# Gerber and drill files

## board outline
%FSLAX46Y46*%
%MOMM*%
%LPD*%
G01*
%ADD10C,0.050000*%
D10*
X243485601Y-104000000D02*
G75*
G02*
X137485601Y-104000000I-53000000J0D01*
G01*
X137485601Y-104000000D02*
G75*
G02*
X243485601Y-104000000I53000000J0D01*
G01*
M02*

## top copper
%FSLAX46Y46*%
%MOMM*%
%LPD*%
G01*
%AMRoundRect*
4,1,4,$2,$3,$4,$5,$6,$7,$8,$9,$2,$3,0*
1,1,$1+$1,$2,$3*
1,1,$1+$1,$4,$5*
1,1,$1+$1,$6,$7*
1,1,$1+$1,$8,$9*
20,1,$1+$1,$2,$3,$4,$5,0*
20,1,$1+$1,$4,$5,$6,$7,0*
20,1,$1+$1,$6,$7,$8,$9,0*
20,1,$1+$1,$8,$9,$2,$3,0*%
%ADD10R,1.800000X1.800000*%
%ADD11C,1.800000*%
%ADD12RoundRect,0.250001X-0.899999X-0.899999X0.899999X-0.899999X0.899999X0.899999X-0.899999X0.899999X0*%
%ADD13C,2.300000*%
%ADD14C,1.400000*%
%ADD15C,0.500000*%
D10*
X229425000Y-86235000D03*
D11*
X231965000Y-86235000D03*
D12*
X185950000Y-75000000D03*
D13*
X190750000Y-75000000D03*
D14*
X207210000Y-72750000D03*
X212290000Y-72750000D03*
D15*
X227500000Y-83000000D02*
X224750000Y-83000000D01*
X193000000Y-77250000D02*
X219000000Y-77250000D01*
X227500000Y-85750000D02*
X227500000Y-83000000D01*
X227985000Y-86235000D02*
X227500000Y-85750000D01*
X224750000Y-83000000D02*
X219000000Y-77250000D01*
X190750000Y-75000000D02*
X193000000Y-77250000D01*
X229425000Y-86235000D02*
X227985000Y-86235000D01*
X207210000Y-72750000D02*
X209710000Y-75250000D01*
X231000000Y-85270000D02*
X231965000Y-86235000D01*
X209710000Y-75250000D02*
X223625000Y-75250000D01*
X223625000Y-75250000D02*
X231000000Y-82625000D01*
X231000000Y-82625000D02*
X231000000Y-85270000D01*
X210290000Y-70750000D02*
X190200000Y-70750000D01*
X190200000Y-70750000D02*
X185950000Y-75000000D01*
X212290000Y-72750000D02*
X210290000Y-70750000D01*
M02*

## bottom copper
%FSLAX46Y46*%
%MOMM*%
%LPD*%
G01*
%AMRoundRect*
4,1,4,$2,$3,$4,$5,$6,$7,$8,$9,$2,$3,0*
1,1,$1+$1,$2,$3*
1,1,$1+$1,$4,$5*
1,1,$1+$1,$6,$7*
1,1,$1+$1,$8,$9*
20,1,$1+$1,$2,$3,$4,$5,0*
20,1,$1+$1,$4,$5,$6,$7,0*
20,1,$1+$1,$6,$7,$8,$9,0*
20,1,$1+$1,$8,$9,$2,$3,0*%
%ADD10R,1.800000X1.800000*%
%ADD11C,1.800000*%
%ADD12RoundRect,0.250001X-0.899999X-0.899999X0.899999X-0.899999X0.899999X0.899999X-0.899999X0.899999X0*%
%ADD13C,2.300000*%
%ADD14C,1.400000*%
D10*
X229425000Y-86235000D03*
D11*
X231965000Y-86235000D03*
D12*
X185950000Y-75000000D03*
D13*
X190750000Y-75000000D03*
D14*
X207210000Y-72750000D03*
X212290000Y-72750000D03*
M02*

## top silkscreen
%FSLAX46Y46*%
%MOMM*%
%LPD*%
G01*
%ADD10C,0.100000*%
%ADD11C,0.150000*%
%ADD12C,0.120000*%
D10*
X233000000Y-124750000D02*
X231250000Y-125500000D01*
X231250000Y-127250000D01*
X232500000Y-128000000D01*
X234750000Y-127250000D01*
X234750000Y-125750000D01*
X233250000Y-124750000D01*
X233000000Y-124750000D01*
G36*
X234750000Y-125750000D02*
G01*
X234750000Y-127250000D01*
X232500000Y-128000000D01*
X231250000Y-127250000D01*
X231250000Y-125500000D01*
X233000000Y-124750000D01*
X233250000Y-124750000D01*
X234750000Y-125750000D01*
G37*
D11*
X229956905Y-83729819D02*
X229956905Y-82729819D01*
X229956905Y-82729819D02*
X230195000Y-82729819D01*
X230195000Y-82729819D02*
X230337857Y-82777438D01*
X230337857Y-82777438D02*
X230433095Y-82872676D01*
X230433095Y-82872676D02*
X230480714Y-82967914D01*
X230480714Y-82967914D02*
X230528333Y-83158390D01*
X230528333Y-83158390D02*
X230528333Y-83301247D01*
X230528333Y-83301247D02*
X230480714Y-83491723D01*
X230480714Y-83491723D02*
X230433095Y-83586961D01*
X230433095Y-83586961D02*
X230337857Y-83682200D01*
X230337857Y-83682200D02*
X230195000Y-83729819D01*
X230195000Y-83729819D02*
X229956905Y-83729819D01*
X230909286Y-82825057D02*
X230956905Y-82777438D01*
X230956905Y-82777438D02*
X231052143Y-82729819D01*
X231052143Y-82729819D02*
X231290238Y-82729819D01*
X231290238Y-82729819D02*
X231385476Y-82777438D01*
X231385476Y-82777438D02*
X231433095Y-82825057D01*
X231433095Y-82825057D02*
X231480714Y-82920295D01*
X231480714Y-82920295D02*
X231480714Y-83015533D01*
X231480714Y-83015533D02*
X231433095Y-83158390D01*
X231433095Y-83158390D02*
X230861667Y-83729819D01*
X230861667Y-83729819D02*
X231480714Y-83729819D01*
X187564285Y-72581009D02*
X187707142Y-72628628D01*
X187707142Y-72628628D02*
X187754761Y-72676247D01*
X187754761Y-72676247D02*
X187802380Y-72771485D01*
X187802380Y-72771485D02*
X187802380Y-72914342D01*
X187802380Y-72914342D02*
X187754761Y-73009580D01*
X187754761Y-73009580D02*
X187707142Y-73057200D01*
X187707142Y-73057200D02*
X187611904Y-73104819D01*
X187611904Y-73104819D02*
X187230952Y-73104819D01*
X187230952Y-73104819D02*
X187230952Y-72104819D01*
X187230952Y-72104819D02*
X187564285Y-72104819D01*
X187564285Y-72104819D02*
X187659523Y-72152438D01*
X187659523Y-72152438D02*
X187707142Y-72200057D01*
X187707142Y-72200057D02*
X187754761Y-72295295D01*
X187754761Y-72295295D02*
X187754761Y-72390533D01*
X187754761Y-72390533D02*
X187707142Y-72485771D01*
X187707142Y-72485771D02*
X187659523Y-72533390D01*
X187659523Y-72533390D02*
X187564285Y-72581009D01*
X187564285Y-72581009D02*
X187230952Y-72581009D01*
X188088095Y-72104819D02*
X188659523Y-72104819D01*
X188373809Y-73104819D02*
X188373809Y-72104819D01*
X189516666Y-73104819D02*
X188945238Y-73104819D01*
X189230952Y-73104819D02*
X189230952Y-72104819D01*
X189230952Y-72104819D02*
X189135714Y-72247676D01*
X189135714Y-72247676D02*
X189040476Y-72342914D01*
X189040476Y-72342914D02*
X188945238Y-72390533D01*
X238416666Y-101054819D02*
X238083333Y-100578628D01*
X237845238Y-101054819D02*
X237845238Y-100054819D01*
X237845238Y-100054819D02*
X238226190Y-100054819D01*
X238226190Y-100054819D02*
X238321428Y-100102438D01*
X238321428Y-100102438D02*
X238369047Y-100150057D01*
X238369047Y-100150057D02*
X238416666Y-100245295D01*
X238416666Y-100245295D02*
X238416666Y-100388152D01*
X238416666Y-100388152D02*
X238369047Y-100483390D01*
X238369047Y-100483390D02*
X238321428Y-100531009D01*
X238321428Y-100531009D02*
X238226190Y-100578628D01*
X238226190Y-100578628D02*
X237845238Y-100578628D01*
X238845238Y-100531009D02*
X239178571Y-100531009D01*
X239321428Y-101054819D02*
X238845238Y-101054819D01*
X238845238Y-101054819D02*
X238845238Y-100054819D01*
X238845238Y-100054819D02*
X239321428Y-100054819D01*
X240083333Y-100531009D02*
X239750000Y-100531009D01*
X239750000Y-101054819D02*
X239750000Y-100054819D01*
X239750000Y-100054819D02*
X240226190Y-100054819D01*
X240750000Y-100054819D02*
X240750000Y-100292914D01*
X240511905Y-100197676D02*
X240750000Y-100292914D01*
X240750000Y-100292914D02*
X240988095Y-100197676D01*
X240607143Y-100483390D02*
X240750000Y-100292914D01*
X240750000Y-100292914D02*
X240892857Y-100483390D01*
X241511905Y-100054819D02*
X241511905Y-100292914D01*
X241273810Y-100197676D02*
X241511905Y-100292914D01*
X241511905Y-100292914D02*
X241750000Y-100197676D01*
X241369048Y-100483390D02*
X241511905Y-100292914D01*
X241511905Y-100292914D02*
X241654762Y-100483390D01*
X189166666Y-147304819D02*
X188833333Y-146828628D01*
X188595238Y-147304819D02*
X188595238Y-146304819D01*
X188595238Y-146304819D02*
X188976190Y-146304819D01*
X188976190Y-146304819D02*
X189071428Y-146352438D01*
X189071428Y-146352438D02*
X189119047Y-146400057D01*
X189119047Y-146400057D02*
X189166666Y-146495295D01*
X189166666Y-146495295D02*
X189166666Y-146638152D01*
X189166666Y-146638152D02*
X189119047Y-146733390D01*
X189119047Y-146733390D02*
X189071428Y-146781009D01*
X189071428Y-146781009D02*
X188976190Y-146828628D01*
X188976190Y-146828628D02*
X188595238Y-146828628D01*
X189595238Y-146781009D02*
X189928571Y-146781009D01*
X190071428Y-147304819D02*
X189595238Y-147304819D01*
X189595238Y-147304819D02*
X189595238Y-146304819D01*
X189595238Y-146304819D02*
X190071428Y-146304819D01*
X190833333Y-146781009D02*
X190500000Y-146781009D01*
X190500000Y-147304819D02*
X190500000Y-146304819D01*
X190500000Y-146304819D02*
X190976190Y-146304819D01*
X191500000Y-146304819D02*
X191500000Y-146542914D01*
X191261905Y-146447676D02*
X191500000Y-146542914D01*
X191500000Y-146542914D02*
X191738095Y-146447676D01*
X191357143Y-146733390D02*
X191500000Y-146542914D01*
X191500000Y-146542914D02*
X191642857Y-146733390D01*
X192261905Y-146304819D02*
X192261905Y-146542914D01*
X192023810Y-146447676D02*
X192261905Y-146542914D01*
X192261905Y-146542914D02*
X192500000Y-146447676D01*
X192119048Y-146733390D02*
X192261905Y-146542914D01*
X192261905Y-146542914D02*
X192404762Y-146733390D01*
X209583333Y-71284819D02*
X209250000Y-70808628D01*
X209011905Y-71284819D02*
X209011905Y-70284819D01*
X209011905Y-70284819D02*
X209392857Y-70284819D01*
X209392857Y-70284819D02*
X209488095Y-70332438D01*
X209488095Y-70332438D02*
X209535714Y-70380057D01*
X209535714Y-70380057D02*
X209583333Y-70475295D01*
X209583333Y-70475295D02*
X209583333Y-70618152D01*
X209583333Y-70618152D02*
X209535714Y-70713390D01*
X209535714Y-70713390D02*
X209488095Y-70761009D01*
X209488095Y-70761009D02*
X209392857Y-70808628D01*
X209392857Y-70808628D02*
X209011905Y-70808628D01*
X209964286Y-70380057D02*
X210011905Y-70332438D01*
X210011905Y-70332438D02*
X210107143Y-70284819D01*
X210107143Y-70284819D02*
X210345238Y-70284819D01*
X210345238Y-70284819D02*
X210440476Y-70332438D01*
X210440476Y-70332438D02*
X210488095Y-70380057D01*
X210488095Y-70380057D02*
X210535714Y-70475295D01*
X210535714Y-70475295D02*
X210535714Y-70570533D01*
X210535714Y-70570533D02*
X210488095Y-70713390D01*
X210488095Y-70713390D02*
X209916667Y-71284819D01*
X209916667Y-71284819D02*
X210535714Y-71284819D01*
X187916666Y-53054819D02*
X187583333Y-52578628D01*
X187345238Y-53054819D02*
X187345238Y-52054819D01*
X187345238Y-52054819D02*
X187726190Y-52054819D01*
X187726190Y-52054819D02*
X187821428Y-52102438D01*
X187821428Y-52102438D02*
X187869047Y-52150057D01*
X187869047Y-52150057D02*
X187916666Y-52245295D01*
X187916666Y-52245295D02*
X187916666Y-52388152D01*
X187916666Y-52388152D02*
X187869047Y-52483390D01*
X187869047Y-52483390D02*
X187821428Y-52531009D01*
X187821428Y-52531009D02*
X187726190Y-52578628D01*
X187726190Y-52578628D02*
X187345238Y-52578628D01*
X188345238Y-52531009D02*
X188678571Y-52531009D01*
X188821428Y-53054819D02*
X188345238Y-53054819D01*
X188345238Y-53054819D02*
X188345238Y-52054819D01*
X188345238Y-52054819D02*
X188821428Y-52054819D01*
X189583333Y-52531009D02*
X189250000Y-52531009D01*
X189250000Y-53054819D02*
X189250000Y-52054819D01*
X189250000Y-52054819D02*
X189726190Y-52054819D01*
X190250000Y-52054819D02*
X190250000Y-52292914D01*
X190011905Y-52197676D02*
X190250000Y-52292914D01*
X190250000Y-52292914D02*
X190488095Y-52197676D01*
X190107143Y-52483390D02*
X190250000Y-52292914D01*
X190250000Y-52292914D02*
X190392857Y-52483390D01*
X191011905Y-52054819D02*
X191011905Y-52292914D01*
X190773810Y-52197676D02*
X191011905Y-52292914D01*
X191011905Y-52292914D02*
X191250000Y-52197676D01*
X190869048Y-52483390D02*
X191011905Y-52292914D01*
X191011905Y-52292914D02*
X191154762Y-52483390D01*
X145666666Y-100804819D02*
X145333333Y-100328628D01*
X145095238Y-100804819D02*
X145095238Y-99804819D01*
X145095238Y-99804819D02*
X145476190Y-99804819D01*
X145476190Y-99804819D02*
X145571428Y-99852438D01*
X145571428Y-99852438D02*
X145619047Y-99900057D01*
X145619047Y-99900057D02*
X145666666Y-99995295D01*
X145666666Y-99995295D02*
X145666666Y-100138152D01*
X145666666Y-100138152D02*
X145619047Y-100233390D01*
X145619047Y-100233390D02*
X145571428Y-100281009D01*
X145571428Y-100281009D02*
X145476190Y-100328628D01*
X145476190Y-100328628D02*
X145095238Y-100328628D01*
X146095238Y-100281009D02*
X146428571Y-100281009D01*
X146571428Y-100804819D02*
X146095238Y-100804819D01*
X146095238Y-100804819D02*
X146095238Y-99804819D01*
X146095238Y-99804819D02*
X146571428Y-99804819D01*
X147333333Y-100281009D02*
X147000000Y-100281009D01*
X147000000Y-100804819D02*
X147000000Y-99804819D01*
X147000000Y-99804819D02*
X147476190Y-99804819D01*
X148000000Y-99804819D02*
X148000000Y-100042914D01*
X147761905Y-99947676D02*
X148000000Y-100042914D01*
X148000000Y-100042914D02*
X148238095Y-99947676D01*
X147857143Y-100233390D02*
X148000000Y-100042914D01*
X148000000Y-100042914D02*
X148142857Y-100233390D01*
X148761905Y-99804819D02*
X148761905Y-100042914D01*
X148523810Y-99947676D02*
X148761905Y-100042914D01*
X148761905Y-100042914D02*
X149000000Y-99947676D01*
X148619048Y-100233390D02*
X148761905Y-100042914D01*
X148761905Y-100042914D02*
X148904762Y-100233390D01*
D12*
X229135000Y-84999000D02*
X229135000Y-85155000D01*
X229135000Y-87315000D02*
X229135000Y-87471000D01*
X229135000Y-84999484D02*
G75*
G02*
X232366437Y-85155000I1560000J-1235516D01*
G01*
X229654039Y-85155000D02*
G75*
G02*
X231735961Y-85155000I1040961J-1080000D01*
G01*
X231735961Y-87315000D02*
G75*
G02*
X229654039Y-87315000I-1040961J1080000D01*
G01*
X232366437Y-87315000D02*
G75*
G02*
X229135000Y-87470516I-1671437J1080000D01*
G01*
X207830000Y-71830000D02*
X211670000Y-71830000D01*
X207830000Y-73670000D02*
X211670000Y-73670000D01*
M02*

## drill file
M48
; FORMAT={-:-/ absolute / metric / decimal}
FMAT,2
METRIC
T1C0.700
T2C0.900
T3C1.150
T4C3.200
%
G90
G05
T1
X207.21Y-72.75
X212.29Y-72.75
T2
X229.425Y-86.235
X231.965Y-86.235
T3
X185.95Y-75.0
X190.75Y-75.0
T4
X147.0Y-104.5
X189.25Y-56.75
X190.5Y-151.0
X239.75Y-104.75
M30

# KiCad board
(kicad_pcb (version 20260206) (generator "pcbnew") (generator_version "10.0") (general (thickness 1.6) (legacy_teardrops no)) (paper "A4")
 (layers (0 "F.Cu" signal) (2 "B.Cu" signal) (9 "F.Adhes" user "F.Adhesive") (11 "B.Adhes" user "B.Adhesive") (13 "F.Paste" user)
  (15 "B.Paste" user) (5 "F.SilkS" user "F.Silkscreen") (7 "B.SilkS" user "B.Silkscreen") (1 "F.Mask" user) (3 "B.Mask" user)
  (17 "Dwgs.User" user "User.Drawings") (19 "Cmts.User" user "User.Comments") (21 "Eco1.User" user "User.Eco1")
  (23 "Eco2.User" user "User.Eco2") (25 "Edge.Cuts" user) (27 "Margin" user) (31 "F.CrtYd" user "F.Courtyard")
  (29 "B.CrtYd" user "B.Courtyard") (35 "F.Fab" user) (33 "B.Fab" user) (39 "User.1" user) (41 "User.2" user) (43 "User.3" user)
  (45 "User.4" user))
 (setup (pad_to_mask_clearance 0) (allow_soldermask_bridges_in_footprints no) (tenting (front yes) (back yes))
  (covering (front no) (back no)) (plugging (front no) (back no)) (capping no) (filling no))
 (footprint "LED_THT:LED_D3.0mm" (layer "F.Cu") (at 229.425 86.235)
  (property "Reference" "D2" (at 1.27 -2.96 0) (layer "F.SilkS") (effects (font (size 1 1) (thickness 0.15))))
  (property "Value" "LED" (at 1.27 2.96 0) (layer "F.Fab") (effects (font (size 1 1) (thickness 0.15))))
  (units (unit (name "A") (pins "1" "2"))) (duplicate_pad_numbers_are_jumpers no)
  (fp_line (start -0.29 -1.236) (end -0.29 -1.08) (stroke (width 0.12) (type solid)) (layer "F.SilkS"))
  (fp_line (start -0.29 1.08) (end -0.29 1.236) (stroke (width 0.12) (type solid)) (layer "F.SilkS"))
  (fp_arc (start -0.29 -1.235516) (mid 1.36566 -1.987699) (end 2.941437 -1.08) (stroke (width 0.12) (type solid)) (layer "F.SilkS"))
  (fp_arc (start 0.229039 -1.08) (mid 1.27 -1.5) (end 2.310961 -1.08) (stroke (width 0.12) (type solid)) (layer "F.SilkS"))
  (fp_arc (start 2.310961 1.08) (mid 1.27 1.5) (end 0.229039 1.08) (stroke (width 0.12) (type solid)) (layer "F.SilkS"))
  (fp_arc (start 2.941437 1.08) (mid 1.36566 1.987699) (end -0.29 1.235516) (stroke (width 0.12) (type solid)) (layer "F.SilkS"))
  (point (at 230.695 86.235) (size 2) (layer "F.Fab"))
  (pad "1" thru_hole rect (at 0 0) (size 1.8 1.8) (drill 0.9) (layers "*.Cu" "*.Mask") (remove_unused_layers no) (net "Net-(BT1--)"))
  (pad "2" thru_hole circle (at 2.54 0) (size 1.8 1.8) (drill 0.9) (layers "*.Cu" "*.Mask") (remove_unused_layers no) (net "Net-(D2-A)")))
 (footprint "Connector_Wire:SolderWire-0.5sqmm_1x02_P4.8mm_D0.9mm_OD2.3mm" (layer "F.Cu") (at 185.95 75)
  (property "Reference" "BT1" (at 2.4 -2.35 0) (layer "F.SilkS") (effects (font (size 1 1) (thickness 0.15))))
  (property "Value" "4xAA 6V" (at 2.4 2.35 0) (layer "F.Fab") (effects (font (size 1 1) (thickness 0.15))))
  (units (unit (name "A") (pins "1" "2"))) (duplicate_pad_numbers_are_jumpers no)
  (pad "1" thru_hole roundrect (at 0 0) (size 2.3 2.3) (drill 1.15) (layers "*.Cu" "*.Mask") (remove_unused_layers no)
   (roundrect_rratio 0.108696) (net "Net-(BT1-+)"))
  (pad "2" thru_hole circle (at 4.8 0) (size 2.3 2.3) (drill 1.15) (layers "*.Cu" "*.Mask") (remove_unused_layers no) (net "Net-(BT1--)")))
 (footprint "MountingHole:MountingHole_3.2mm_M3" (layer "F.Cu") (at 239.75 104.75)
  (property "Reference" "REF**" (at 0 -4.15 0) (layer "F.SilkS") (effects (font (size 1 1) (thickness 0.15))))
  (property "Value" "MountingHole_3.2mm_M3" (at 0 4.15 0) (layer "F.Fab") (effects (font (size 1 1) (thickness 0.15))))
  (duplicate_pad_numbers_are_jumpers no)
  (pad "" np_thru_hole circle (at 0 0) (size 3.2 3.2) (drill 3.2) (layers "*.Cu" "*.Mask")))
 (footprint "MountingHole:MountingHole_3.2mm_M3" (layer "F.Cu") (at 190.5 151)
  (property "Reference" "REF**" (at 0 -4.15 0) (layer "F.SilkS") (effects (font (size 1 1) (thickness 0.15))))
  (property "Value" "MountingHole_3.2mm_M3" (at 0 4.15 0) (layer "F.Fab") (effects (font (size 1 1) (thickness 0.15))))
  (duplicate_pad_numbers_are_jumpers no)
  (pad "" np_thru_hole circle (at 0 0) (size 3.2 3.2) (drill 3.2) (layers "*.Cu" "*.Mask")))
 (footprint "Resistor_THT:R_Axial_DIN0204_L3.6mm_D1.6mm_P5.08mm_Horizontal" (layer "F.Cu") (at 207.21 72.75)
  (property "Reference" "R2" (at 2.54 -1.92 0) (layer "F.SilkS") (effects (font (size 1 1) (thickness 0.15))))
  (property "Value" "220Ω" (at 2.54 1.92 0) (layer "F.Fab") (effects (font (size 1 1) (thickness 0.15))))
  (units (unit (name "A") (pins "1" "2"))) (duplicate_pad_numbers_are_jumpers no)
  (fp_line (start 0.62 -0.92) (end 4.46 -0.92) (stroke (width 0.12) (type solid)) (layer "F.SilkS"))
  (fp_line (start 0.62 0.92) (end 4.46 0.92) (stroke (width 0.12) (type solid)) (layer "F.SilkS"))
  (pad "1" thru_hole circle (at 0 0) (size 1.4 1.4) (drill 0.7) (layers "*.Cu" "*.Mask") (remove_unused_layers no) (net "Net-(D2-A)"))
  (pad "2" thru_hole circle (at 5.08 0) (size 1.4 1.4) (drill 0.7) (layers "*.Cu" "*.Mask") (remove_unused_layers no) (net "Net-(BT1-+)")))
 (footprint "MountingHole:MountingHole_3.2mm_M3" (layer "F.Cu") (at 189.25 56.75)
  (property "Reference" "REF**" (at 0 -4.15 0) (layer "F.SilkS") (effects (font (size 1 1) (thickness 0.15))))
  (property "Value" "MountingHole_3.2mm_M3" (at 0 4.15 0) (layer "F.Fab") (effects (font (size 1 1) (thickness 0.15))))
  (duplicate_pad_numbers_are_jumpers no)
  (pad "" np_thru_hole circle (at 0 0) (size 3.2 3.2) (drill 3.2) (layers "*.Cu" "*.Mask")))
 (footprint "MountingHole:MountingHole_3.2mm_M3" (layer "F.Cu") (at 147 104.5)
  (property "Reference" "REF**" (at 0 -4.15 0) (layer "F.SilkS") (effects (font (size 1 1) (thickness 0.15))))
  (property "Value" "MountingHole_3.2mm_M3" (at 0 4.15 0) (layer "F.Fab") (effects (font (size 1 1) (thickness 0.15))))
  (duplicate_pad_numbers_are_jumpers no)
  (pad "" np_thru_hole circle (at 0 0) (size 3.2 3.2) (drill 3.2) (layers "*.Cu" "*.Mask")))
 (gr_poly
  (pts (xy 233 124.75) (xy 231.25 125.5) (xy 231.25 127.25) (xy 232.5 128) (xy 234.75 127.25) (xy 234.75 125.75) (xy 233.25 124.75))
  (stroke (width 0.1) (type solid)) (fill yes) (layer "F.SilkS"))
 (gr_circle (center 190.485601 104) (end 243.485601 104) (stroke (width 0.05) (type solid)) (fill no) (layer "Edge.Cuts"))
 (segment (start 227.5 83) (end 224.75 83) (width 0.5) (layer "F.Cu") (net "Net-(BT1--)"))
 (segment (start 193 77.25) (end 219 77.25) (width 0.5) (layer "F.Cu") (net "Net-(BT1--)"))
 (segment (start 227.5 85.75) (end 227.5 83) (width 0.5) (layer "F.Cu") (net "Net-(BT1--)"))
 (segment (start 227.985 86.235) (end 227.5 85.75) (width 0.5) (layer "F.Cu") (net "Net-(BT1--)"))
 (segment (start 224.75 83) (end 219 77.25) (width 0.5) (layer "F.Cu") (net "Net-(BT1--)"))
 (segment (start 190.75 75) (end 193 77.25) (width 0.5) (layer "F.Cu") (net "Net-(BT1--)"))
 (segment (start 229.425 86.235) (end 227.985 86.235) (width 0.5) (layer "F.Cu") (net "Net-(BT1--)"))
 (segment (start 207.21 72.75) (end 209.71 75.25) (width 0.5) (layer "F.Cu") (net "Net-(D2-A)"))
 (segment (start 231 85.27) (end 231.965 86.235) (width 0.5) (layer "F.Cu") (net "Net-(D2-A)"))
 (segment (start 209.71 75.25) (end 223.625 75.25) (width 0.5) (layer "F.Cu") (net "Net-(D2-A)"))
 (segment (start 223.625 75.25) (end 231 82.625) (width 0.5) (layer "F.Cu") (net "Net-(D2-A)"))
 (segment (start 231 82.625) (end 231 85.27) (width 0.5) (layer "F.Cu") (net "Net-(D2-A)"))
 (segment (start 210.29 70.75) (end 190.2 70.75) (width 0.5) (layer "F.Cu") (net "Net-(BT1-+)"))
 (segment (start 190.2 70.75) (end 185.95 75) (width 0.5) (layer "F.Cu") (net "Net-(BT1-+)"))
 (segment (start 212.29 72.75) (end 210.29 70.75) (width 0.5) (layer "F.Cu") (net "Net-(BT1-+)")))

